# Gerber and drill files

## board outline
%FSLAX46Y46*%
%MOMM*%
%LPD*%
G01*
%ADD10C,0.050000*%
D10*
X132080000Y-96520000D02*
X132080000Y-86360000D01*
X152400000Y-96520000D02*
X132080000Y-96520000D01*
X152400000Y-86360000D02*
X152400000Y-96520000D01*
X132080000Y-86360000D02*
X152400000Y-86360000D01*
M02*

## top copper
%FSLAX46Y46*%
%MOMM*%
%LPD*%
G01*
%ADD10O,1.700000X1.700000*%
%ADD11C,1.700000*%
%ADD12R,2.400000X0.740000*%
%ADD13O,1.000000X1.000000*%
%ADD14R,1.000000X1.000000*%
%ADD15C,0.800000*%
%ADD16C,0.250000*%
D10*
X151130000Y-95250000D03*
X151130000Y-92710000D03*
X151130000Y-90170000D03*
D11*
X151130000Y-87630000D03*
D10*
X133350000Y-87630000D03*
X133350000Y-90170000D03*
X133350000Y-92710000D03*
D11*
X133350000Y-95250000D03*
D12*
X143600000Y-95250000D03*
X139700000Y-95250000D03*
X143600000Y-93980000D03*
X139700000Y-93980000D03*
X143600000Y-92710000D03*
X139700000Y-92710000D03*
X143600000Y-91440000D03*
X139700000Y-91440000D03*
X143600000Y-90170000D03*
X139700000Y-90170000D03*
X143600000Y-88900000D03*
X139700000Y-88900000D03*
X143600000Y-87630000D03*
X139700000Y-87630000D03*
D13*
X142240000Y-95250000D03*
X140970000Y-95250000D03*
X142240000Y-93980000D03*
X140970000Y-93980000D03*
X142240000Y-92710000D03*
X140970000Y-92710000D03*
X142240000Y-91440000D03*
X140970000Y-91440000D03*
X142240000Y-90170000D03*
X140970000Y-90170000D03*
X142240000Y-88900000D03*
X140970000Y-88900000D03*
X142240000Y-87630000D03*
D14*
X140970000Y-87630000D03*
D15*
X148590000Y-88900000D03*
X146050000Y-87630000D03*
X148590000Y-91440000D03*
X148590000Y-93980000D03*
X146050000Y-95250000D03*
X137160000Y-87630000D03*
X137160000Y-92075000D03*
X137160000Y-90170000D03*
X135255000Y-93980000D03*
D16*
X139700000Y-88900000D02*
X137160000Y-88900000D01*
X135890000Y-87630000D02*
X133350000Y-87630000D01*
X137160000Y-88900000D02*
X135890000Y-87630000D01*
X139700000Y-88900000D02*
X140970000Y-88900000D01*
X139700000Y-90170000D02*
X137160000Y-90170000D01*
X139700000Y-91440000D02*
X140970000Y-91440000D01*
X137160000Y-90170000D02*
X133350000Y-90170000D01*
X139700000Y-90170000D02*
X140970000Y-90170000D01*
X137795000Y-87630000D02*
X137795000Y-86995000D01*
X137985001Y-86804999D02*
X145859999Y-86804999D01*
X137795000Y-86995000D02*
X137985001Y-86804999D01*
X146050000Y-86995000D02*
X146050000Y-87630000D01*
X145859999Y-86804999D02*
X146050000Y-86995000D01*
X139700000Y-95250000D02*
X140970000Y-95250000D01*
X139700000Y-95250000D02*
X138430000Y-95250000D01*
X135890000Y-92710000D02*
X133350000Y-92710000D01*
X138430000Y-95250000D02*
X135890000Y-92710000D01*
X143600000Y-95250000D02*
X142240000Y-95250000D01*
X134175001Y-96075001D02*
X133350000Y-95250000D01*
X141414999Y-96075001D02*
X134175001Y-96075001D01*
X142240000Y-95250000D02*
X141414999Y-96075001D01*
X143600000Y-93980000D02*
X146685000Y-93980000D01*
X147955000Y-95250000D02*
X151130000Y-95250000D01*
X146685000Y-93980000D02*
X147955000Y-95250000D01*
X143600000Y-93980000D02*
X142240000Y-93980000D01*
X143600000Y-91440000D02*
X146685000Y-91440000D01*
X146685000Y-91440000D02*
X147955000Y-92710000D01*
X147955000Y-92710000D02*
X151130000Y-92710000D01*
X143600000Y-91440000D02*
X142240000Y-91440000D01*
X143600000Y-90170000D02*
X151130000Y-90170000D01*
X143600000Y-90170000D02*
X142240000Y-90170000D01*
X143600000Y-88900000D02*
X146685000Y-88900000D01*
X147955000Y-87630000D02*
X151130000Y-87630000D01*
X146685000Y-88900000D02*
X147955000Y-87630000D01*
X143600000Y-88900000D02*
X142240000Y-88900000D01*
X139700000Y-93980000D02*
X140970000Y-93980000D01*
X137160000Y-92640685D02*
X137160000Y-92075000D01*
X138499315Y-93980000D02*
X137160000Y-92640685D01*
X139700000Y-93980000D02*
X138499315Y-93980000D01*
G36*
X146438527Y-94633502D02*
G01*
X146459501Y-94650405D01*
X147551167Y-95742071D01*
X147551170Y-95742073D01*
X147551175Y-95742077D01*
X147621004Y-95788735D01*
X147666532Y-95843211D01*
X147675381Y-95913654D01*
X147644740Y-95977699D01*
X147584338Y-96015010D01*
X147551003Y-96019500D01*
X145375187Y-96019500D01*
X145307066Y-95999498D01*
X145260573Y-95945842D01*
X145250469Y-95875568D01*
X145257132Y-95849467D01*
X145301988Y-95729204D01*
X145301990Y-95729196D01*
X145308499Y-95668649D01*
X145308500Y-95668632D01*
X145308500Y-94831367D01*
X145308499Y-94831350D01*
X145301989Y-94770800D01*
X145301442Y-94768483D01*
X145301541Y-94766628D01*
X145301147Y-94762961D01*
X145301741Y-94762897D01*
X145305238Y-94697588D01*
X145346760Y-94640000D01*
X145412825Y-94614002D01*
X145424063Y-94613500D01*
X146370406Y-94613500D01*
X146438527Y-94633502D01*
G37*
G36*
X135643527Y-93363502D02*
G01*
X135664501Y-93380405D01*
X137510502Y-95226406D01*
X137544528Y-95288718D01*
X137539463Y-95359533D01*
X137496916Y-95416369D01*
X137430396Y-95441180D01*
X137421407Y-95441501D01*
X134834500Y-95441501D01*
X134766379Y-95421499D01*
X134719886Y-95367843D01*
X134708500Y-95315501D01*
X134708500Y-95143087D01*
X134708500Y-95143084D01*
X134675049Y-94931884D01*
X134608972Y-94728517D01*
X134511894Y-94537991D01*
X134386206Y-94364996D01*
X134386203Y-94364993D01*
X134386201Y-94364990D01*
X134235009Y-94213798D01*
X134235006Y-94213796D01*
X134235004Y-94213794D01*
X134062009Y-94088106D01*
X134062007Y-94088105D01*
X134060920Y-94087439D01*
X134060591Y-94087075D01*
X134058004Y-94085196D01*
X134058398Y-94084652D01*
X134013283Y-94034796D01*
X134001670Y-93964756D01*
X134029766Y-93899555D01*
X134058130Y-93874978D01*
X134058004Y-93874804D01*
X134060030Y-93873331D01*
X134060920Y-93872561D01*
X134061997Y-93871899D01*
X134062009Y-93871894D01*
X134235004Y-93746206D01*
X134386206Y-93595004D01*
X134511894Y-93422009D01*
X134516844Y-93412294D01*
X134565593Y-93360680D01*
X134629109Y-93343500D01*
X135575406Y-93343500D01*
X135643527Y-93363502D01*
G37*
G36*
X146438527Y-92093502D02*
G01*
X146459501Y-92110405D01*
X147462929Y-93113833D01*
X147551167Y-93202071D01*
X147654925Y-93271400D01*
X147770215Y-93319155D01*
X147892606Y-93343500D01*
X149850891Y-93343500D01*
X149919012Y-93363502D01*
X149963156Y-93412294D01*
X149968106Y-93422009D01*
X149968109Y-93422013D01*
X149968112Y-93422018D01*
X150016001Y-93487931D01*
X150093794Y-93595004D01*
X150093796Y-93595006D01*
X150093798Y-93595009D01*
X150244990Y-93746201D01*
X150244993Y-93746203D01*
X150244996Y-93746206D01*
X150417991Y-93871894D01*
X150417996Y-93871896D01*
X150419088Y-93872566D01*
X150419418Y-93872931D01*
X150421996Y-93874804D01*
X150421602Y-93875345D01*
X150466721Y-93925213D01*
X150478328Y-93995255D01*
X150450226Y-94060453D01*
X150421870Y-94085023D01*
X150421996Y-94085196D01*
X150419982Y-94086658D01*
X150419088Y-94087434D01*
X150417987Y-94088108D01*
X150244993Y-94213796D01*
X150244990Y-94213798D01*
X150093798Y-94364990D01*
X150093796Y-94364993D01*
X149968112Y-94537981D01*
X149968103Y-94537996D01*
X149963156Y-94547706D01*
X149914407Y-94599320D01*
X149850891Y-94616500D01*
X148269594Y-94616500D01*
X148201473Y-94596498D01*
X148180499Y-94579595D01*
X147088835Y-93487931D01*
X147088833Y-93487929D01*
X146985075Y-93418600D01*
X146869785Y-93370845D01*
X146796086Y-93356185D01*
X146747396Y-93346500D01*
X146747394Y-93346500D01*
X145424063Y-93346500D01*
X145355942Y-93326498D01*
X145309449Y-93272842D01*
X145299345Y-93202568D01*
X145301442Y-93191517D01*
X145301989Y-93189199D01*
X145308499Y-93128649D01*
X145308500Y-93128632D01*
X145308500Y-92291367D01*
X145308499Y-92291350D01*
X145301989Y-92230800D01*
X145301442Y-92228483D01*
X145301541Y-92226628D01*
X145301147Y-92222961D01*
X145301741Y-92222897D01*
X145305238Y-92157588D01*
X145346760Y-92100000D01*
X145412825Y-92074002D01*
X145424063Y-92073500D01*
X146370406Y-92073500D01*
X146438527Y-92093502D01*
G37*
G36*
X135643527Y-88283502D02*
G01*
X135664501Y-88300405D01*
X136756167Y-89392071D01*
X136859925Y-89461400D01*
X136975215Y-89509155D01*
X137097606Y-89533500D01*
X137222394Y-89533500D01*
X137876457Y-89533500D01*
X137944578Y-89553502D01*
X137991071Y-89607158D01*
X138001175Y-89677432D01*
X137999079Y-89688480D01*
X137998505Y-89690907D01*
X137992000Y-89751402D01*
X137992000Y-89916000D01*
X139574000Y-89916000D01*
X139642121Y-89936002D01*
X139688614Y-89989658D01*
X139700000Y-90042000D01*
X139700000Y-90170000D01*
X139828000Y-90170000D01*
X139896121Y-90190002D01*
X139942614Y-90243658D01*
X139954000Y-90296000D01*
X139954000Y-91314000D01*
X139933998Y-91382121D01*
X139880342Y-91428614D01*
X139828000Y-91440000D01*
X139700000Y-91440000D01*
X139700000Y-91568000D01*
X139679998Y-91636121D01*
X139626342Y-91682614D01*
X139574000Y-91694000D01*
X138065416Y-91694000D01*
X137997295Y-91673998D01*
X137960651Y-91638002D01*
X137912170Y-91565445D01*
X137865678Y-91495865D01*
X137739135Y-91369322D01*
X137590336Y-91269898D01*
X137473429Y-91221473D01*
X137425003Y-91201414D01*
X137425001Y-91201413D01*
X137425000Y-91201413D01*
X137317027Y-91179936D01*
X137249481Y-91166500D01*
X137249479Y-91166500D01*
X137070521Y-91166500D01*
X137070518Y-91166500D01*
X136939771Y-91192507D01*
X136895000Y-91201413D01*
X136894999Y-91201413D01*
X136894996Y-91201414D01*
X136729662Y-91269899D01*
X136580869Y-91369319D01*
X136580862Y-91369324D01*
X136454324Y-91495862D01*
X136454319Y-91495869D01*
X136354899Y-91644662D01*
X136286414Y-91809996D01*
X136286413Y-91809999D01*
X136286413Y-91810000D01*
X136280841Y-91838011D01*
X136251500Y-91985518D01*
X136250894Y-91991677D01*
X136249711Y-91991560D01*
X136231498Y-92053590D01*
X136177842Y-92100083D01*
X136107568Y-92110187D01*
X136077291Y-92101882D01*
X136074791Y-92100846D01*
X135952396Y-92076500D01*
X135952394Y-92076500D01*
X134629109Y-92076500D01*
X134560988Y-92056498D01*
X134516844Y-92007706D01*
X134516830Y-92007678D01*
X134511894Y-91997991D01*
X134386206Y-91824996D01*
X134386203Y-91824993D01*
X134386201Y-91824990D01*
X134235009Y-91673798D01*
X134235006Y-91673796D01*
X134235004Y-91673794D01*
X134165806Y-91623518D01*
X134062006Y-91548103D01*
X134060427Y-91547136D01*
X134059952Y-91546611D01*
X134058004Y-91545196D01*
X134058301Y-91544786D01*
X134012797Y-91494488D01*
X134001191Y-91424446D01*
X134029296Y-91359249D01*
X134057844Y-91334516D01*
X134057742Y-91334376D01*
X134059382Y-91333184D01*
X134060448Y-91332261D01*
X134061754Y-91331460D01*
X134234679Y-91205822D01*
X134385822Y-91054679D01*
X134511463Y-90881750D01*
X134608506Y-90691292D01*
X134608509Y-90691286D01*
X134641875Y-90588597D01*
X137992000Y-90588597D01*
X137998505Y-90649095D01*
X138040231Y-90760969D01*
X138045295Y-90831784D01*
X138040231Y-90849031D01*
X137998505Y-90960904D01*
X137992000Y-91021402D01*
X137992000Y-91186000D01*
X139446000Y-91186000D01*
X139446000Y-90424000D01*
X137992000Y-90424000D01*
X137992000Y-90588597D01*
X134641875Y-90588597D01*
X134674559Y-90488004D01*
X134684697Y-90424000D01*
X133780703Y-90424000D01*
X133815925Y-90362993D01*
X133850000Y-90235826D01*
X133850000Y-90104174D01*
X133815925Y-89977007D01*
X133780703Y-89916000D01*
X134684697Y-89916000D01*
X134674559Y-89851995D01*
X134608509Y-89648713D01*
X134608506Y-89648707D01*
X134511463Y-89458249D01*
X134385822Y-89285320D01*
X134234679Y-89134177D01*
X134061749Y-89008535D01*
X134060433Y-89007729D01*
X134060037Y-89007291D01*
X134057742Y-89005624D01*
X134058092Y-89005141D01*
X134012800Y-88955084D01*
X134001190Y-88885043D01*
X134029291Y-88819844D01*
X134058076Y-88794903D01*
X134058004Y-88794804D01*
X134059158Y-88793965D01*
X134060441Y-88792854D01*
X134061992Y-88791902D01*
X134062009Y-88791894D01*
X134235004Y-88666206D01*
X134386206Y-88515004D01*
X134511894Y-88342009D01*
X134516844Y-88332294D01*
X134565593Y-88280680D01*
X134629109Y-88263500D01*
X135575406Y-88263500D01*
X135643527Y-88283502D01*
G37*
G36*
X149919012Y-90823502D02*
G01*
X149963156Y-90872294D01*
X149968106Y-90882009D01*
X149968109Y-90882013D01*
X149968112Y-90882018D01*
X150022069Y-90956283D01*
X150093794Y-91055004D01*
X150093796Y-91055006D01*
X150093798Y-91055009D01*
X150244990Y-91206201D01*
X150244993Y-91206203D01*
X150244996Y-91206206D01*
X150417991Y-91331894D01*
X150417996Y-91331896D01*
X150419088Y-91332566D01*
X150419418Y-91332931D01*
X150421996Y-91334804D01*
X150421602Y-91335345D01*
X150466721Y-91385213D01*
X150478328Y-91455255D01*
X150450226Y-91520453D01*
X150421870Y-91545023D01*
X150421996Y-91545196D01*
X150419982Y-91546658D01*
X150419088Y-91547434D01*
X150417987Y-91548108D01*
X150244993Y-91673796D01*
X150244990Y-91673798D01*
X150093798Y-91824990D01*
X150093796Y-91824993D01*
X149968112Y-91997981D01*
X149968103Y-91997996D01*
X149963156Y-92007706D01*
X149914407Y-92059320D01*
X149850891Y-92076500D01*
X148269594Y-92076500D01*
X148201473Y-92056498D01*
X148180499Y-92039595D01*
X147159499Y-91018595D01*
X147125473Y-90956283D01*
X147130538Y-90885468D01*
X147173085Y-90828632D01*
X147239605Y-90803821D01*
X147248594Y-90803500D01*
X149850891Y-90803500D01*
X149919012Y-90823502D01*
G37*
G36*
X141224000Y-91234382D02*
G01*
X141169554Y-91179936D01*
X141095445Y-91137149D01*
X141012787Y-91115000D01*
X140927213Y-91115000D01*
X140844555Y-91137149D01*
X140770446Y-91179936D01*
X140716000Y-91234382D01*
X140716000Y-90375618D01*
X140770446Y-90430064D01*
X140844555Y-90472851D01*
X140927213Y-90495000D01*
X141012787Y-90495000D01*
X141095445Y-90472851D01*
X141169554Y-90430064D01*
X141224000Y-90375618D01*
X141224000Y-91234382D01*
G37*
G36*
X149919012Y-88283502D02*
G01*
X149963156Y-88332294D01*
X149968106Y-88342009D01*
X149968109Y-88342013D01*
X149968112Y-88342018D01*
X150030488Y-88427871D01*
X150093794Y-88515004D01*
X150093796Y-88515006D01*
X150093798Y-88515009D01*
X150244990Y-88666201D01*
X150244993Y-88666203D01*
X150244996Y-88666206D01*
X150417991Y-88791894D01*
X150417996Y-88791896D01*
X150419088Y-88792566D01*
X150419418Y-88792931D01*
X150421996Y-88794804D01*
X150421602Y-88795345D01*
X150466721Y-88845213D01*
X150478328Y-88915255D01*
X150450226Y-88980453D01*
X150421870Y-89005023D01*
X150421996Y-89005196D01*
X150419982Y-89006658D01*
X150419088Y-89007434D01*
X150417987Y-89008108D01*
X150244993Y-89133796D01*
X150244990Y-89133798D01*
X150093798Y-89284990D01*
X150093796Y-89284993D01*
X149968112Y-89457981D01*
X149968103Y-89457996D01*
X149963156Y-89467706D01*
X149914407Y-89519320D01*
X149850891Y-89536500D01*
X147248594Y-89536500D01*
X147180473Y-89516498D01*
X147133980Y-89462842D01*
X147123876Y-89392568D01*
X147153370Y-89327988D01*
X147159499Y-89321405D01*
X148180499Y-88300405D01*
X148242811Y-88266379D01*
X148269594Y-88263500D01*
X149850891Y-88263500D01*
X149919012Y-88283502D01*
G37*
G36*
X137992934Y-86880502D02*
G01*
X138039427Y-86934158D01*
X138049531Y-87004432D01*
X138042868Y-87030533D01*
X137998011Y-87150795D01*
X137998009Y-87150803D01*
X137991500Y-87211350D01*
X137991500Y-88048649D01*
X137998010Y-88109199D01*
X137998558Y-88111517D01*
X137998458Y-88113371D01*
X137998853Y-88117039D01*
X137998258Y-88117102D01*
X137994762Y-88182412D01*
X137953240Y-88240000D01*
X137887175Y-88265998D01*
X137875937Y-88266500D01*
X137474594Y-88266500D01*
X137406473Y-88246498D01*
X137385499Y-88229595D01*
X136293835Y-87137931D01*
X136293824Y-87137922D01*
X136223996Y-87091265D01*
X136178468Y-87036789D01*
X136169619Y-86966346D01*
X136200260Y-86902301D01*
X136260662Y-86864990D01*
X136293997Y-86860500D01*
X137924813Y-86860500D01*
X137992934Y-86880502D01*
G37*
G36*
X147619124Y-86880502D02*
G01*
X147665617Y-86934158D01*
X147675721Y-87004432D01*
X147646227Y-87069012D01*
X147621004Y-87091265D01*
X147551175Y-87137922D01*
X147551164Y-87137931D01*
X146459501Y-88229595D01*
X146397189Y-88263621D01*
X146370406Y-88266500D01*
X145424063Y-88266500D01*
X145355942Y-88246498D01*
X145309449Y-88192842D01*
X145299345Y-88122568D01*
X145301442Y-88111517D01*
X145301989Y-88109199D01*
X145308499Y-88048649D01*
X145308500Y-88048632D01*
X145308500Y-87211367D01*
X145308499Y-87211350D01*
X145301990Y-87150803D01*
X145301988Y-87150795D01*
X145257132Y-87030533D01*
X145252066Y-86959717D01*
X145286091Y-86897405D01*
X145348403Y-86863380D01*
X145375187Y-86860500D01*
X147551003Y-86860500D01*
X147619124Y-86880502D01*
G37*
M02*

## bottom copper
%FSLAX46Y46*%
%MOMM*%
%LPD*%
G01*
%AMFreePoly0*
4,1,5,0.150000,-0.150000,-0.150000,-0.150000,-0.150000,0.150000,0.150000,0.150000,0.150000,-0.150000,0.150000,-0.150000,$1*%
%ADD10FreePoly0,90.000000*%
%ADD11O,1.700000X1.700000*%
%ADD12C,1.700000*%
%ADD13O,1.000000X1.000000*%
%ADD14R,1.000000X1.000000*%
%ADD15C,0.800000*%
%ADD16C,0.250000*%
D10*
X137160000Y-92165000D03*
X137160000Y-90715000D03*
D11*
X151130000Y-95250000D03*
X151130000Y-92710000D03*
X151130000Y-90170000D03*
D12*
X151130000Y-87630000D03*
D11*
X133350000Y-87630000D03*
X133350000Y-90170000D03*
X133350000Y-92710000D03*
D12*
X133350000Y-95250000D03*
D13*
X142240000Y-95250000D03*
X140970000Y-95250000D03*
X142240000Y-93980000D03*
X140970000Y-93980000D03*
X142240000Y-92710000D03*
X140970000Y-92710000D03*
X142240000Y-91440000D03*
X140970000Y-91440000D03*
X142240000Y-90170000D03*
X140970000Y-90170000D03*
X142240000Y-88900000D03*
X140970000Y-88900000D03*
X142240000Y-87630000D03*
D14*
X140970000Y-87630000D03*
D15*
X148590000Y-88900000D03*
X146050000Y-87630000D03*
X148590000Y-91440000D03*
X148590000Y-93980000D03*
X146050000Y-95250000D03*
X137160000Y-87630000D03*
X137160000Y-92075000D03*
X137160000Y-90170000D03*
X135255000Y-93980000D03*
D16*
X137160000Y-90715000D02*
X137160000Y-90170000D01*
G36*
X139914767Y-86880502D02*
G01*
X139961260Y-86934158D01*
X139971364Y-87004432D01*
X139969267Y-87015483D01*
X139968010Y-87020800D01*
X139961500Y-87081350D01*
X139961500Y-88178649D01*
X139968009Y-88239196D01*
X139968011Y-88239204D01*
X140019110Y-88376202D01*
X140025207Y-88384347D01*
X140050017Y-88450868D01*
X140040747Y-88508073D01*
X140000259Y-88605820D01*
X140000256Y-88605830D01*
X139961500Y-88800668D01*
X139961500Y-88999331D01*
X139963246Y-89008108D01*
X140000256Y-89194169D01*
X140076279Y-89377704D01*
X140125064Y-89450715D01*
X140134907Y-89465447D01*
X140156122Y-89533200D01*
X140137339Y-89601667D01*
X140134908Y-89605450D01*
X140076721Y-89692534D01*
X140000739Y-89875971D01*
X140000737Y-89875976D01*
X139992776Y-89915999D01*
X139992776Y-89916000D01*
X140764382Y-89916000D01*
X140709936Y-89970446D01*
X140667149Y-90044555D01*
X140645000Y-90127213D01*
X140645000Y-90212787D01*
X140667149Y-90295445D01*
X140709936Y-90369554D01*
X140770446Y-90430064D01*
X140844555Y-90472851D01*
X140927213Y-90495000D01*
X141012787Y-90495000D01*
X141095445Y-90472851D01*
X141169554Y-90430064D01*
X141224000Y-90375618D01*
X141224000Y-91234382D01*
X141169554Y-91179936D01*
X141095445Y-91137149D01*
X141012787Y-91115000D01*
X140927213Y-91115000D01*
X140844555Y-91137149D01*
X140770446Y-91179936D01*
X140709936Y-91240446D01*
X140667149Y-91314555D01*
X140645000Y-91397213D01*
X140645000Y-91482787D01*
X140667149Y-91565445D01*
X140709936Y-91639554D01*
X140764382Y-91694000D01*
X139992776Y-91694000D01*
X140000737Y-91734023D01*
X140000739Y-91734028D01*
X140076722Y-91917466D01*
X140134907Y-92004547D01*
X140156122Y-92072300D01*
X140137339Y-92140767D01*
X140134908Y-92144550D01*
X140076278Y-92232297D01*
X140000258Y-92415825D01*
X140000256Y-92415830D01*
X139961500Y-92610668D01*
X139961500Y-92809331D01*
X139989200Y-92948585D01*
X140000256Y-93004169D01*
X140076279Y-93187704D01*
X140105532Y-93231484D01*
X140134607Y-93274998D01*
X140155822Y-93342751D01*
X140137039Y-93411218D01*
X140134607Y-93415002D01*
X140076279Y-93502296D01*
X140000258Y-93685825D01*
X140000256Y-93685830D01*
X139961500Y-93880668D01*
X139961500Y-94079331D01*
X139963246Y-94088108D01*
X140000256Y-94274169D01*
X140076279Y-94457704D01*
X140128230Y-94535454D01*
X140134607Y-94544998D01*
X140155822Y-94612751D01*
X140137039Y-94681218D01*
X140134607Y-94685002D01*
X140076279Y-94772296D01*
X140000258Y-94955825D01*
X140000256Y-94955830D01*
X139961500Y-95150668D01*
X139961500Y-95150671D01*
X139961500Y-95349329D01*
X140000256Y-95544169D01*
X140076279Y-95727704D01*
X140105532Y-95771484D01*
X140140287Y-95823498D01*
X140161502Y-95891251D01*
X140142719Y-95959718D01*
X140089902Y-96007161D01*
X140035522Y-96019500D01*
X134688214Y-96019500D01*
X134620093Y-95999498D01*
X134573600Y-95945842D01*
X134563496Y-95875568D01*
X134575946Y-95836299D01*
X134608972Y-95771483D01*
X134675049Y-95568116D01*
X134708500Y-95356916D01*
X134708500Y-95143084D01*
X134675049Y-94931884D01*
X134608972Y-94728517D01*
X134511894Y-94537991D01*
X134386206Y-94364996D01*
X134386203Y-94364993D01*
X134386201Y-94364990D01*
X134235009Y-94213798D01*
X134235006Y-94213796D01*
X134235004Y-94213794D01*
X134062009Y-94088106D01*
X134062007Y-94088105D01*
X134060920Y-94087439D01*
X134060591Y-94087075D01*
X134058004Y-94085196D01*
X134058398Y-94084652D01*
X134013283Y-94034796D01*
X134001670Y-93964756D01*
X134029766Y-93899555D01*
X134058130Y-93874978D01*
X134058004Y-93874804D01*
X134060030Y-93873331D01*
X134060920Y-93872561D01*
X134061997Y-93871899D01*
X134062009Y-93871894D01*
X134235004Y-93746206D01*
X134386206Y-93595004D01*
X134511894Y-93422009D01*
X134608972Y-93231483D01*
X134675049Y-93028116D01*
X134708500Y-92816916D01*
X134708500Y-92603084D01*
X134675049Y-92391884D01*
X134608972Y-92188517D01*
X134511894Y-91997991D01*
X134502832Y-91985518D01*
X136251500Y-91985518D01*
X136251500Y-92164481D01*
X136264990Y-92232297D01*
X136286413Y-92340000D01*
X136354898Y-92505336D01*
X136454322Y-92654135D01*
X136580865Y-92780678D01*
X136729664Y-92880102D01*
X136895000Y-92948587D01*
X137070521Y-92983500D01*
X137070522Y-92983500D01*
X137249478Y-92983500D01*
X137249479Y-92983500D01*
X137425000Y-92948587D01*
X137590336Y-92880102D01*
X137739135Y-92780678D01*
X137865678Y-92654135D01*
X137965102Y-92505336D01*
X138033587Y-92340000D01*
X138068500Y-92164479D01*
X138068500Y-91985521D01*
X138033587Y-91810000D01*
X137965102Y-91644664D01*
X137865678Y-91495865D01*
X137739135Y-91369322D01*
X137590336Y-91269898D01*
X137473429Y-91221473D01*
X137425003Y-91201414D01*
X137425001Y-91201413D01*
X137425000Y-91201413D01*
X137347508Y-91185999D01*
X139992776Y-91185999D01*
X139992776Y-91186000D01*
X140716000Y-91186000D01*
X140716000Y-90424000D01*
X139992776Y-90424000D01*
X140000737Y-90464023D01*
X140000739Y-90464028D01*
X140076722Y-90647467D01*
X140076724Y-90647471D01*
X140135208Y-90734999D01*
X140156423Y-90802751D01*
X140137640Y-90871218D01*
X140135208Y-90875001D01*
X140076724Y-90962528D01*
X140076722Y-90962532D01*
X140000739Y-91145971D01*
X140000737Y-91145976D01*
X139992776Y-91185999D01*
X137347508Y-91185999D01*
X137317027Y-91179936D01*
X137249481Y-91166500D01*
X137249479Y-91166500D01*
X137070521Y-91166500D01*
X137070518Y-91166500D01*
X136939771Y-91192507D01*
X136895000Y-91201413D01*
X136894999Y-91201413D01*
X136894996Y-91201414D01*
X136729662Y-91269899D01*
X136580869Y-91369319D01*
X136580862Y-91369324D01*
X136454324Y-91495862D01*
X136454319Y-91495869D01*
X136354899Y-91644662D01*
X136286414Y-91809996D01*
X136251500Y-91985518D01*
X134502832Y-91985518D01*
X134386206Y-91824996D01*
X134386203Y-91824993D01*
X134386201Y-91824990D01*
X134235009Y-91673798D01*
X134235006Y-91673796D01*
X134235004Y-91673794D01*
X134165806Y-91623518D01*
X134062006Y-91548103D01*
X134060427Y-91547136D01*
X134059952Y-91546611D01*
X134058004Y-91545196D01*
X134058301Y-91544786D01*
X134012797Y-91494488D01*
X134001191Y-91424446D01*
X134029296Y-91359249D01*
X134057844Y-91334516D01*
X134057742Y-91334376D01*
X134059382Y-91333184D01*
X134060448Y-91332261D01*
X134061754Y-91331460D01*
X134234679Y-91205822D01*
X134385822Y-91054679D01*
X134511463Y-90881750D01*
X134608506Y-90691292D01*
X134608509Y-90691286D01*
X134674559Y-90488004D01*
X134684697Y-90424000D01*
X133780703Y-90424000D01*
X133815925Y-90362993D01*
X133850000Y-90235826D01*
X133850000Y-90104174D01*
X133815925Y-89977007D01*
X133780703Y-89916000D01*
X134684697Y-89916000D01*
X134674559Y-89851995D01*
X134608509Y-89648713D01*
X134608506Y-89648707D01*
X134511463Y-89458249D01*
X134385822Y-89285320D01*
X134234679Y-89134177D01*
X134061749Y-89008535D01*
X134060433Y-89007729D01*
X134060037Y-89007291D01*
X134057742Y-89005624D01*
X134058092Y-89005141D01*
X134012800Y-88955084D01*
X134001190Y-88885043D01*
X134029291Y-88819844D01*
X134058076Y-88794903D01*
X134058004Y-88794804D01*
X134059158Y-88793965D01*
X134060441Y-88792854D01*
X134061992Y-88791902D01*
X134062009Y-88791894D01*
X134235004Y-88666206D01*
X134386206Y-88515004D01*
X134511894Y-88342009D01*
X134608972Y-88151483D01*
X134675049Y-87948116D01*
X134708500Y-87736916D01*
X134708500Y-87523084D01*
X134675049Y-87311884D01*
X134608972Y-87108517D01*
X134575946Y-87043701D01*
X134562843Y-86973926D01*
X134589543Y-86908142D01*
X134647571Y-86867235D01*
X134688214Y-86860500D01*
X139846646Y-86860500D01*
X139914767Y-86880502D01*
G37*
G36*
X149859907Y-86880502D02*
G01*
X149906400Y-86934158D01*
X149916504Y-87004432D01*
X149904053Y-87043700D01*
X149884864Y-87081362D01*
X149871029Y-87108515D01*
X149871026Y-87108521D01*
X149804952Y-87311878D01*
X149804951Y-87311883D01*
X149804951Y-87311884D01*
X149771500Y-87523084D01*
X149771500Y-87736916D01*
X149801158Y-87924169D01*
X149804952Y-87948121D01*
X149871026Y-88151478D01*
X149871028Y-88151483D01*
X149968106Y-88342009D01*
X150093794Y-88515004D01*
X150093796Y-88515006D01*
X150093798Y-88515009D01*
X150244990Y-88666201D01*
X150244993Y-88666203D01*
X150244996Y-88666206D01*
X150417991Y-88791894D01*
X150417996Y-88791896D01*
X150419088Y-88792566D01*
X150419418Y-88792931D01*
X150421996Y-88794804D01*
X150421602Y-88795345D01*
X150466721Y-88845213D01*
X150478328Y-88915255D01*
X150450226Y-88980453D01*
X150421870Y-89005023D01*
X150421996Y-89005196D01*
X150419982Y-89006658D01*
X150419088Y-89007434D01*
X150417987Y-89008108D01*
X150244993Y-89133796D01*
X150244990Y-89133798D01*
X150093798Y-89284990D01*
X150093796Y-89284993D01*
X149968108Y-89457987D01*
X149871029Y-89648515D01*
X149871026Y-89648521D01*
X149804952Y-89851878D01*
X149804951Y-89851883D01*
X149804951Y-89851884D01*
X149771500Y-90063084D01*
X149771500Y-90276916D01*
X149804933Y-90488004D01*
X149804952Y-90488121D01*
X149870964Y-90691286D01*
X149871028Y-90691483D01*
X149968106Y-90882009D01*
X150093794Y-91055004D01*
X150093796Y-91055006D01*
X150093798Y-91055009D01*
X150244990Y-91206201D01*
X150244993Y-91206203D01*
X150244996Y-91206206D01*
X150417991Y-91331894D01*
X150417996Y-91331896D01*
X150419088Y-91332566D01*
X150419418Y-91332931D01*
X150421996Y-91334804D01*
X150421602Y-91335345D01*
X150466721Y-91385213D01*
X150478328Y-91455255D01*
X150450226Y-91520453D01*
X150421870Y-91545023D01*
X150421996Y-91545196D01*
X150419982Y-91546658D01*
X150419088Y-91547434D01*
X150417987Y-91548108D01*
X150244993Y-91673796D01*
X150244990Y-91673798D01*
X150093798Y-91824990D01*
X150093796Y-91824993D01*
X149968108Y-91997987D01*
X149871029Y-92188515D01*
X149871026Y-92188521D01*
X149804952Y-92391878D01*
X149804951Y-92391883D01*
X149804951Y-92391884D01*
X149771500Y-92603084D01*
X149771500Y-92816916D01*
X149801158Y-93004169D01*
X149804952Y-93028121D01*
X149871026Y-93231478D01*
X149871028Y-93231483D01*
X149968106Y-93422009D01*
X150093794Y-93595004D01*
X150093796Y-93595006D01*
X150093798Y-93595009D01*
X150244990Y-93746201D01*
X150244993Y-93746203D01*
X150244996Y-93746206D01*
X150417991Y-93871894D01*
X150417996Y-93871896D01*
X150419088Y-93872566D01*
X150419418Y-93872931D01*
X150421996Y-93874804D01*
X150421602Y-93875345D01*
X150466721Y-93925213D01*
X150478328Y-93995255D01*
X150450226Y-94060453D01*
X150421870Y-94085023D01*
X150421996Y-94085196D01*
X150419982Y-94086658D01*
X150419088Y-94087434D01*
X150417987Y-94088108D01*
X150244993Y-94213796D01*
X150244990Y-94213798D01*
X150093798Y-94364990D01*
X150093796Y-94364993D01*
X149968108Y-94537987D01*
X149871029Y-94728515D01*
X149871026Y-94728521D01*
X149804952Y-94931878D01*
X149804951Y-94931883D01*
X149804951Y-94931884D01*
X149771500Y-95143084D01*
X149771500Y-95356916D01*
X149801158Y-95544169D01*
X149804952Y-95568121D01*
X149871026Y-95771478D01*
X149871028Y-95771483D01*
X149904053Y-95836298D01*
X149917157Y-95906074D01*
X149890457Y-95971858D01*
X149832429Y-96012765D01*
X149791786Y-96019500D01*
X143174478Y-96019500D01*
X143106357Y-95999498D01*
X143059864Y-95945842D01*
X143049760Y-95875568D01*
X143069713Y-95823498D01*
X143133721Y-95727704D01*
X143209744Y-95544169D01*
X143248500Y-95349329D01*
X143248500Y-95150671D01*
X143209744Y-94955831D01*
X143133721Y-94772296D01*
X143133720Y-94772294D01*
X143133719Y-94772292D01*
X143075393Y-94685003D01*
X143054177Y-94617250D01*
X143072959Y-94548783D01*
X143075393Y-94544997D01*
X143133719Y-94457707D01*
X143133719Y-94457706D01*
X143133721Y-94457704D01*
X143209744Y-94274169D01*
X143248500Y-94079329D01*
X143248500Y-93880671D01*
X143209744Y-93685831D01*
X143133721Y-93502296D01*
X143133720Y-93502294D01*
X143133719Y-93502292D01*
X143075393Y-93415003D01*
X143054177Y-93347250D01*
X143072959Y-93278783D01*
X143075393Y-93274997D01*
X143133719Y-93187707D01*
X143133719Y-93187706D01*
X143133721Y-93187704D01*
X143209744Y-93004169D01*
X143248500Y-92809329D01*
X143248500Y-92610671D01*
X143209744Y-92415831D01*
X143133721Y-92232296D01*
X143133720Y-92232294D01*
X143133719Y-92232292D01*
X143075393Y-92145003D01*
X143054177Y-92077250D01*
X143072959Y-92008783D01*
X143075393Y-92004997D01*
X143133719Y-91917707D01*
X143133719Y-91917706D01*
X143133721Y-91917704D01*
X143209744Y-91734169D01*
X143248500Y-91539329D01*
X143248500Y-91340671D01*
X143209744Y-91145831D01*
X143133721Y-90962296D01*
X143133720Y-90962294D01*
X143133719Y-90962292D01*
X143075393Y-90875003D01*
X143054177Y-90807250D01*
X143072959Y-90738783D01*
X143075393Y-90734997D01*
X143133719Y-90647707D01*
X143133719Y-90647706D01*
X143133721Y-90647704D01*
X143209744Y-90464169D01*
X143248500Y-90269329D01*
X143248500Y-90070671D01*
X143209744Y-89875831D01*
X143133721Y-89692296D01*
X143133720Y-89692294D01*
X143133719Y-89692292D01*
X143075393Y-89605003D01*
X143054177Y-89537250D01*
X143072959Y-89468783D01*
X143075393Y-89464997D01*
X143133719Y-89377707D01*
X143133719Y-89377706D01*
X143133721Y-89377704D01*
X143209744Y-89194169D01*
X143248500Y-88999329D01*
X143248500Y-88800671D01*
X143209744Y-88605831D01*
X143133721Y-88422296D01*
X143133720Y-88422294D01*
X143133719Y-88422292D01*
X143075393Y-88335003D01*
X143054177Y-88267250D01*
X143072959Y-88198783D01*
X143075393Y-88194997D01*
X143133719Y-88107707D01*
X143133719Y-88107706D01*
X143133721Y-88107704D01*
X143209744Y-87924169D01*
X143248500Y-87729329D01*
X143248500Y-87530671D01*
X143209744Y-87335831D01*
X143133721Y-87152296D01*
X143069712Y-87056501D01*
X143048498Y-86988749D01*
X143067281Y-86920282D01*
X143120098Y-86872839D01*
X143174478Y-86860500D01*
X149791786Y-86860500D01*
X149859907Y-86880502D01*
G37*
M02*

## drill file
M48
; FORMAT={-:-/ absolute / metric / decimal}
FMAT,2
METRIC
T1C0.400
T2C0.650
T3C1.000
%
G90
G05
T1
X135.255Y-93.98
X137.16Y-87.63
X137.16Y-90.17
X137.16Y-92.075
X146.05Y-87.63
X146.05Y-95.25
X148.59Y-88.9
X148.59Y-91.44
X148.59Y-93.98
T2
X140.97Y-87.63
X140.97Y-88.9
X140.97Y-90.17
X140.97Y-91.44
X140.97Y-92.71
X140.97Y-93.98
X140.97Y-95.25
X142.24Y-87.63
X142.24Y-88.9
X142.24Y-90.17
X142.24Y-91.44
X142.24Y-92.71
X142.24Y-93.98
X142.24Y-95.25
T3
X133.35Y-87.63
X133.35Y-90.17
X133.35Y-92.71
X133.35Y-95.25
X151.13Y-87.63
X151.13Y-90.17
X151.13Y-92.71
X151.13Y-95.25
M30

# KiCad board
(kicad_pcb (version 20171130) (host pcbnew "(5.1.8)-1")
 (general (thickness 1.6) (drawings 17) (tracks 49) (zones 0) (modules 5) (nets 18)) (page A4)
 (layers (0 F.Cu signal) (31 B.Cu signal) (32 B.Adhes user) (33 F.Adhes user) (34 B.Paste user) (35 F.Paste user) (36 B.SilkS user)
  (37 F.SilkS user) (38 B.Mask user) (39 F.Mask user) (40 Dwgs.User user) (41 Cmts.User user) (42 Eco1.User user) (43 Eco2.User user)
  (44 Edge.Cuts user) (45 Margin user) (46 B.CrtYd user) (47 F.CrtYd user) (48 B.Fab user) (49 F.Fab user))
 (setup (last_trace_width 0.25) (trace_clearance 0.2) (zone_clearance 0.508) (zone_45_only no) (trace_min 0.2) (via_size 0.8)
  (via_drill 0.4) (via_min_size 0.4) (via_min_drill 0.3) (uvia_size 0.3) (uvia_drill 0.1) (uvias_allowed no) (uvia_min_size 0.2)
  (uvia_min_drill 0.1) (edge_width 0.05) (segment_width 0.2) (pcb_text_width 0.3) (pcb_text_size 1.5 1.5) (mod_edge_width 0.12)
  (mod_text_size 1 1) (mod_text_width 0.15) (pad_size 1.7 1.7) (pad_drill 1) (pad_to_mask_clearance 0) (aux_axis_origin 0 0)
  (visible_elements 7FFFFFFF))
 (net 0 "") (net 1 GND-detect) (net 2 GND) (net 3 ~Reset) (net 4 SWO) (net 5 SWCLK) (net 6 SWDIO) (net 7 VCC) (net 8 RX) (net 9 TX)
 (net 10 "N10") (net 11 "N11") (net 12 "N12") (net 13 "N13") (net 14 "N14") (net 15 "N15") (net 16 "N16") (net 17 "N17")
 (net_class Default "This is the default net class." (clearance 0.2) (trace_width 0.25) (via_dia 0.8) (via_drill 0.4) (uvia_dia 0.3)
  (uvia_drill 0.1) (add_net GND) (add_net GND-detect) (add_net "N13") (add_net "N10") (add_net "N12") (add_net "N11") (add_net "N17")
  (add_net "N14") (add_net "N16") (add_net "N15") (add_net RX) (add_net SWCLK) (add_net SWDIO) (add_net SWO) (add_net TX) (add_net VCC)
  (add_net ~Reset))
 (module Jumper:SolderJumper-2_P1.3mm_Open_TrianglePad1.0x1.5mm (layer B.Cu) (at 137.16 91.44 90)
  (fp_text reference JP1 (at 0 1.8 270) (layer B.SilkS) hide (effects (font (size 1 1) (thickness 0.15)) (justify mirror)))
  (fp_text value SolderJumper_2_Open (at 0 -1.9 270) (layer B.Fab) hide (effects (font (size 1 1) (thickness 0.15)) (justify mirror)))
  (pad 1 smd custom (at -0.725 0 90) (size 0.3 0.3) (layers B.Cu B.Mask) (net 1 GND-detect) (zone_connect 2)
   (options (clearance outline) (anchor rect)) (primitives))
  (pad 2 smd custom (at 0.725 0 90) (size 0.3 0.3) (layers B.Cu B.Mask) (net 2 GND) (zone_connect 2)
   (options (clearance outline) (anchor rect)) (primitives)))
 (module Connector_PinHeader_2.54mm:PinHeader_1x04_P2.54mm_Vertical (layer B.Cu) (at 151.13 87.63 180)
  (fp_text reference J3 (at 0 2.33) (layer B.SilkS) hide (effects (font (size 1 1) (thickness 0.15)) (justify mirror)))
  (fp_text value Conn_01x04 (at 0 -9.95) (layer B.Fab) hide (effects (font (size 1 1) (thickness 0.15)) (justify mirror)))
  (pad 4 thru_hole oval (at 0 -7.62 180) (size 1.7 1.7) (drill 1) (layers *.Cu *.Mask) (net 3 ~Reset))
  (pad 3 thru_hole oval (at 0 -5.08 180) (size 1.7 1.7) (drill 1) (layers *.Cu *.Mask) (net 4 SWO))
  (pad 2 thru_hole oval (at 0 -2.54 180) (size 1.7 1.7) (drill 1) (layers *.Cu *.Mask) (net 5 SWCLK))
  (pad 1 thru_hole circle (at 0 0 180) (size 1.7 1.7) (drill 1) (layers *.Cu *.Mask) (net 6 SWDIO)))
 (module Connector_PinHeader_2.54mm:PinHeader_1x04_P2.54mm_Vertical (layer B.Cu) (at 133.35 95.25)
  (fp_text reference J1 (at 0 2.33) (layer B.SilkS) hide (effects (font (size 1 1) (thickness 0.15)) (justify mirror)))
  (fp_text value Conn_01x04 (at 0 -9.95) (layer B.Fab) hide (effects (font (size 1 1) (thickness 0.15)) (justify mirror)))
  (pad 4 thru_hole oval (at 0 -7.62) (size 1.7 1.7) (drill 1) (layers *.Cu *.Mask) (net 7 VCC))
  (pad 3 thru_hole oval (at 0 -5.08) (size 1.7 1.7) (drill 1) (layers *.Cu *.Mask) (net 2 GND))
  (pad 2 thru_hole oval (at 0 -2.54) (size 1.7 1.7) (drill 1) (layers *.Cu *.Mask) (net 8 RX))
  (pad 1 thru_hole circle (at 0 0) (size 1.7 1.7) (drill 1) (layers *.Cu *.Mask) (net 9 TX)))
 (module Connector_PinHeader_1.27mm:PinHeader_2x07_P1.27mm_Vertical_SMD (layer F.Cu) (at 141.65 91.44)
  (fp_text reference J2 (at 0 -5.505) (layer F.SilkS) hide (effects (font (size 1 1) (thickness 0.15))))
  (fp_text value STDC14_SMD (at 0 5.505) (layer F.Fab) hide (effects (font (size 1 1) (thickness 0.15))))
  (pad 14 smd rect (at 1.95 3.81) (size 2.4 0.74) (layers F.Cu F.Paste F.Mask) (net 9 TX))
  (pad 13 smd rect (at -1.95 3.81) (size 2.4 0.74) (layers F.Cu F.Paste F.Mask) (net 8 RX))
  (pad 12 smd rect (at 1.95 2.54) (size 2.4 0.74) (layers F.Cu F.Paste F.Mask) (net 3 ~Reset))
  (pad 11 smd rect (at -1.95 2.54) (size 2.4 0.74) (layers F.Cu F.Paste F.Mask) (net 1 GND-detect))
  (pad 10 smd rect (at 1.95 1.27) (size 2.4 0.74) (layers F.Cu F.Paste F.Mask) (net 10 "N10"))
  (pad 9 smd rect (at -1.95 1.27) (size 2.4 0.74) (layers F.Cu F.Paste F.Mask) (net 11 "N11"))
  (pad 8 smd rect (at 1.95 0) (size 2.4 0.74) (layers F.Cu F.Paste F.Mask) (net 4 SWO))
  (pad 7 smd rect (at -1.95 0) (size 2.4 0.74) (layers F.Cu F.Paste F.Mask) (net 2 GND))
  (pad 6 smd rect (at 1.95 -1.27) (size 2.4 0.74) (layers F.Cu F.Paste F.Mask) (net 5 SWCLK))
  (pad 5 smd rect (at -1.95 -1.27) (size 2.4 0.74) (layers F.Cu F.Paste F.Mask) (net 2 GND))
  (pad 4 smd rect (at 1.95 -2.54) (size 2.4 0.74) (layers F.Cu F.Paste F.Mask) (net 6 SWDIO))
  (pad 3 smd rect (at -1.95 -2.54) (size 2.4 0.74) (layers F.Cu F.Paste F.Mask) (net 7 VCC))
  (pad 2 smd rect (at 1.95 -3.81) (size 2.4 0.74) (layers F.Cu F.Paste F.Mask) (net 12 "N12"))
  (pad 1 smd rect (at -1.95 -3.81) (size 2.4 0.74) (layers F.Cu F.Paste F.Mask) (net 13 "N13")))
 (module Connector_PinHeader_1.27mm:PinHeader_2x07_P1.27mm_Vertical (layer F.Cu) (at 140.97 87.63)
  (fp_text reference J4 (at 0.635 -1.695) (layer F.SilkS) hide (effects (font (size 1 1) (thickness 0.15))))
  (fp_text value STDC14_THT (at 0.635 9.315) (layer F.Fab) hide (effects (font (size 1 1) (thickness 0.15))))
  (pad 14 thru_hole oval (at 1.27 7.62) (size 1 1) (drill 0.65) (layers *.Cu *.Mask) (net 9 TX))
  (pad 13 thru_hole oval (at 0 7.62) (size 1 1) (drill 0.65) (layers *.Cu *.Mask) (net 8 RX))
  (pad 12 thru_hole oval (at 1.27 6.35) (size 1 1) (drill 0.65) (layers *.Cu *.Mask) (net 3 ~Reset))
  (pad 11 thru_hole oval (at 0 6.35) (size 1 1) (drill 0.65) (layers *.Cu *.Mask) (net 1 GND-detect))
  (pad 10 thru_hole oval (at 1.27 5.08) (size 1 1) (drill 0.65) (layers *.Cu *.Mask) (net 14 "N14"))
  (pad 9 thru_hole oval (at 0 5.08) (size 1 1) (drill 0.65) (layers *.Cu *.Mask) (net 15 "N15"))
  (pad 8 thru_hole oval (at 1.27 3.81) (size 1 1) (drill 0.65) (layers *.Cu *.Mask) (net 4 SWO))
  (pad 7 thru_hole oval (at 0 3.81) (size 1 1) (drill 0.65) (layers *.Cu *.Mask) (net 2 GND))
  (pad 6 thru_hole oval (at 1.27 2.54) (size 1 1) (drill 0.65) (layers *.Cu *.Mask) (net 5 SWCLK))
  (pad 5 thru_hole oval (at 0 2.54) (size 1 1) (drill 0.65) (layers *.Cu *.Mask) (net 2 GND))
  (pad 4 thru_hole oval (at 1.27 1.27) (size 1 1) (drill 0.65) (layers *.Cu *.Mask) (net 6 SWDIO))
  (pad 3 thru_hole oval (at 0 1.27) (size 1 1) (drill 0.65) (layers *.Cu *.Mask) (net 7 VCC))
  (pad 2 thru_hole oval (at 1.27 0) (size 1 1) (drill 0.65) (layers *.Cu *.Mask) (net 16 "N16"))
  (pad 1 thru_hole rect (at 0 0) (size 1 1) (drill 0.65) (layers *.Cu *.Mask) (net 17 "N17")))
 (gr_line (start 132.08 96.52) (end 132.08 86.36) (layer Edge.Cuts) (width 0.05))
 (gr_line (start 152.4 96.52) (end 132.08 96.52) (layer Edge.Cuts) (width 0.05))
 (gr_line (start 152.4 86.36) (end 152.4 96.52) (layer Edge.Cuts) (width 0.05))
 (gr_line (start 132.08 86.36) (end 152.4 86.36) (layer Edge.Cuts) (width 0.05))
 (via (at 148.59 88.9) (size 0.8) (drill 0.4) (layers F.Cu B.Cu) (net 2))
 (via (at 146.05 87.63) (size 0.8) (drill 0.4) (layers F.Cu B.Cu) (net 2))
 (via (at 148.59 91.44) (size 0.8) (drill 0.4) (layers F.Cu B.Cu) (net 2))
 (via (at 148.59 93.98) (size 0.8) (drill 0.4) (layers F.Cu B.Cu) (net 2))
 (via (at 146.05 95.25) (size 0.8) (drill 0.4) (layers F.Cu B.Cu) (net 2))
 (via (at 137.16 87.63) (size 0.8) (drill 0.4) (layers F.Cu B.Cu) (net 2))
 (via (at 137.16 92.075) (size 0.8) (drill 0.4) (layers F.Cu B.Cu) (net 1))
 (segment (start 139.7 88.9) (end 137.16 88.9) (width 0.25) (layer F.Cu) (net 7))
 (segment (start 135.89 87.63) (end 133.35 87.63) (width 0.25) (layer F.Cu) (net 7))
 (segment (start 137.16 88.9) (end 135.89 87.63) (width 0.25) (layer F.Cu) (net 7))
 (segment (start 139.7 88.9) (end 140.97 88.9) (width 0.25) (layer F.Cu) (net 7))
 (segment (start 139.7 90.17) (end 137.16 90.17) (width 0.25) (layer F.Cu) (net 2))
 (segment (start 139.7 91.44) (end 140.97 91.44) (width 0.25) (layer F.Cu) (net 2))
 (segment (start 137.16 90.17) (end 133.35 90.17) (width 0.25) (layer F.Cu) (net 2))
 (via (at 137.16 90.17) (size 0.8) (drill 0.4) (layers F.Cu B.Cu) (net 2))
 (segment (start 137.16 90.715) (end 137.16 90.17) (width 0.25) (layer B.Cu) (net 2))
 (segment (start 139.7 90.17) (end 140.97 90.17) (width 0.25) (layer F.Cu) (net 2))
 (segment (start 137.795 87.63) (end 137.795 86.995) (width 0.25) (layer F.Cu) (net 2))
 (segment (start 137.985001 86.804999) (end 145.859999 86.804999) (width 0.25) (layer F.Cu) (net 2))
 (segment (start 137.795 86.995) (end 137.985001 86.804999) (width 0.25) (layer F.Cu) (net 2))
 (segment (start 146.05 86.995) (end 146.05 87.63) (width 0.25) (layer F.Cu) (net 2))
 (segment (start 145.859999 86.804999) (end 146.05 86.995) (width 0.25) (layer F.Cu) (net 2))
 (via (at 135.255 93.98) (size 0.8) (drill 0.4) (layers F.Cu B.Cu) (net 2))
 (segment (start 139.7 95.25) (end 140.97 95.25) (width 0.25) (layer F.Cu) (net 8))
 (segment (start 139.7 95.25) (end 138.43 95.25) (width 0.25) (layer F.Cu) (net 8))
 (segment (start 135.89 92.71) (end 133.35 92.71) (width 0.25) (layer F.Cu) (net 8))
 (segment (start 138.43 95.25) (end 135.89 92.71) (width 0.25) (layer F.Cu) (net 8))
 (segment (start 143.6 95.25) (end 142.24 95.25) (width 0.25) (layer F.Cu) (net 9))
 (segment (start 134.175001 96.075001) (end 133.35 95.25) (width 0.25) (layer F.Cu) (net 9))
 (segment (start 141.414999 96.075001) (end 134.175001 96.075001) (width 0.25) (layer F.Cu) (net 9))
 (segment (start 142.24 95.25) (end 141.414999 96.075001) (width 0.25) (layer F.Cu) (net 9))
 (segment (start 143.6 93.98) (end 146.685 93.98) (width 0.25) (layer F.Cu) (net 3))
 (segment (start 147.955 95.25) (end 151.13 95.25) (width 0.25) (layer F.Cu) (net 3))
 (segment (start 146.685 93.98) (end 147.955 95.25) (width 0.25) (layer F.Cu) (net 3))
 (segment (start 143.6 93.98) (end 142.24 93.98) (width 0.25) (layer F.Cu) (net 3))
 (segment (start 143.6 91.44) (end 146.685 91.44) (width 0.25) (layer F.Cu) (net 4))
 (segment (start 146.685 91.44) (end 147.955 92.71) (width 0.25) (layer F.Cu) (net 4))
 (segment (start 147.955 92.71) (end 151.13 92.71) (width 0.25) (layer F.Cu) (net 4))
 (segment (start 143.6 91.44) (end 142.24 91.44) (width 0.25) (layer F.Cu) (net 4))
 (segment (start 143.6 90.17) (end 151.13 90.17) (width 0.25) (layer F.Cu) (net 5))
 (segment (start 143.6 90.17) (end 142.24 90.17) (width 0.25) (layer F.Cu) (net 5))
 (segment (start 143.6 88.9) (end 146.685 88.9) (width 0.25) (layer F.Cu) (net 6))
 (segment (start 147.955 87.63) (end 151.13 87.63) (width 0.25) (layer F.Cu) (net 6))
 (segment (start 146.685 88.9) (end 147.955 87.63) (width 0.25) (layer F.Cu) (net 6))
 (segment (start 143.6 88.9) (end 142.24 88.9) (width 0.25) (layer F.Cu) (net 6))
 (segment (start 139.7 93.98) (end 140.97 93.98) (width 0.25) (layer F.Cu) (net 1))
 (segment (start 137.16 92.640685) (end 137.16 92.075) (width 0.25) (layer F.Cu) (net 1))
 (segment (start 138.499315 93.98) (end 137.16 92.640685) (width 0.25) (layer F.Cu) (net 1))
 (segment (start 139.7 93.98) (end 138.499315 93.98) (width 0.25) (layer F.Cu) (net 1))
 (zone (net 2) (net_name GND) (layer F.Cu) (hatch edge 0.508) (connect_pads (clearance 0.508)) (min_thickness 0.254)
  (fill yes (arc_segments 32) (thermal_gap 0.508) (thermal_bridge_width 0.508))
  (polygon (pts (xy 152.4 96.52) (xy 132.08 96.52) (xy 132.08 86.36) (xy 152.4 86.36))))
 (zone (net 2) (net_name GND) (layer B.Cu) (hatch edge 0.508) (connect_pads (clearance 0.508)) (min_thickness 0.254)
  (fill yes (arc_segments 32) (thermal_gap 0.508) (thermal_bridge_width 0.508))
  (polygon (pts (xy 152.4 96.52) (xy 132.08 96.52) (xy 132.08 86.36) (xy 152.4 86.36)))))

